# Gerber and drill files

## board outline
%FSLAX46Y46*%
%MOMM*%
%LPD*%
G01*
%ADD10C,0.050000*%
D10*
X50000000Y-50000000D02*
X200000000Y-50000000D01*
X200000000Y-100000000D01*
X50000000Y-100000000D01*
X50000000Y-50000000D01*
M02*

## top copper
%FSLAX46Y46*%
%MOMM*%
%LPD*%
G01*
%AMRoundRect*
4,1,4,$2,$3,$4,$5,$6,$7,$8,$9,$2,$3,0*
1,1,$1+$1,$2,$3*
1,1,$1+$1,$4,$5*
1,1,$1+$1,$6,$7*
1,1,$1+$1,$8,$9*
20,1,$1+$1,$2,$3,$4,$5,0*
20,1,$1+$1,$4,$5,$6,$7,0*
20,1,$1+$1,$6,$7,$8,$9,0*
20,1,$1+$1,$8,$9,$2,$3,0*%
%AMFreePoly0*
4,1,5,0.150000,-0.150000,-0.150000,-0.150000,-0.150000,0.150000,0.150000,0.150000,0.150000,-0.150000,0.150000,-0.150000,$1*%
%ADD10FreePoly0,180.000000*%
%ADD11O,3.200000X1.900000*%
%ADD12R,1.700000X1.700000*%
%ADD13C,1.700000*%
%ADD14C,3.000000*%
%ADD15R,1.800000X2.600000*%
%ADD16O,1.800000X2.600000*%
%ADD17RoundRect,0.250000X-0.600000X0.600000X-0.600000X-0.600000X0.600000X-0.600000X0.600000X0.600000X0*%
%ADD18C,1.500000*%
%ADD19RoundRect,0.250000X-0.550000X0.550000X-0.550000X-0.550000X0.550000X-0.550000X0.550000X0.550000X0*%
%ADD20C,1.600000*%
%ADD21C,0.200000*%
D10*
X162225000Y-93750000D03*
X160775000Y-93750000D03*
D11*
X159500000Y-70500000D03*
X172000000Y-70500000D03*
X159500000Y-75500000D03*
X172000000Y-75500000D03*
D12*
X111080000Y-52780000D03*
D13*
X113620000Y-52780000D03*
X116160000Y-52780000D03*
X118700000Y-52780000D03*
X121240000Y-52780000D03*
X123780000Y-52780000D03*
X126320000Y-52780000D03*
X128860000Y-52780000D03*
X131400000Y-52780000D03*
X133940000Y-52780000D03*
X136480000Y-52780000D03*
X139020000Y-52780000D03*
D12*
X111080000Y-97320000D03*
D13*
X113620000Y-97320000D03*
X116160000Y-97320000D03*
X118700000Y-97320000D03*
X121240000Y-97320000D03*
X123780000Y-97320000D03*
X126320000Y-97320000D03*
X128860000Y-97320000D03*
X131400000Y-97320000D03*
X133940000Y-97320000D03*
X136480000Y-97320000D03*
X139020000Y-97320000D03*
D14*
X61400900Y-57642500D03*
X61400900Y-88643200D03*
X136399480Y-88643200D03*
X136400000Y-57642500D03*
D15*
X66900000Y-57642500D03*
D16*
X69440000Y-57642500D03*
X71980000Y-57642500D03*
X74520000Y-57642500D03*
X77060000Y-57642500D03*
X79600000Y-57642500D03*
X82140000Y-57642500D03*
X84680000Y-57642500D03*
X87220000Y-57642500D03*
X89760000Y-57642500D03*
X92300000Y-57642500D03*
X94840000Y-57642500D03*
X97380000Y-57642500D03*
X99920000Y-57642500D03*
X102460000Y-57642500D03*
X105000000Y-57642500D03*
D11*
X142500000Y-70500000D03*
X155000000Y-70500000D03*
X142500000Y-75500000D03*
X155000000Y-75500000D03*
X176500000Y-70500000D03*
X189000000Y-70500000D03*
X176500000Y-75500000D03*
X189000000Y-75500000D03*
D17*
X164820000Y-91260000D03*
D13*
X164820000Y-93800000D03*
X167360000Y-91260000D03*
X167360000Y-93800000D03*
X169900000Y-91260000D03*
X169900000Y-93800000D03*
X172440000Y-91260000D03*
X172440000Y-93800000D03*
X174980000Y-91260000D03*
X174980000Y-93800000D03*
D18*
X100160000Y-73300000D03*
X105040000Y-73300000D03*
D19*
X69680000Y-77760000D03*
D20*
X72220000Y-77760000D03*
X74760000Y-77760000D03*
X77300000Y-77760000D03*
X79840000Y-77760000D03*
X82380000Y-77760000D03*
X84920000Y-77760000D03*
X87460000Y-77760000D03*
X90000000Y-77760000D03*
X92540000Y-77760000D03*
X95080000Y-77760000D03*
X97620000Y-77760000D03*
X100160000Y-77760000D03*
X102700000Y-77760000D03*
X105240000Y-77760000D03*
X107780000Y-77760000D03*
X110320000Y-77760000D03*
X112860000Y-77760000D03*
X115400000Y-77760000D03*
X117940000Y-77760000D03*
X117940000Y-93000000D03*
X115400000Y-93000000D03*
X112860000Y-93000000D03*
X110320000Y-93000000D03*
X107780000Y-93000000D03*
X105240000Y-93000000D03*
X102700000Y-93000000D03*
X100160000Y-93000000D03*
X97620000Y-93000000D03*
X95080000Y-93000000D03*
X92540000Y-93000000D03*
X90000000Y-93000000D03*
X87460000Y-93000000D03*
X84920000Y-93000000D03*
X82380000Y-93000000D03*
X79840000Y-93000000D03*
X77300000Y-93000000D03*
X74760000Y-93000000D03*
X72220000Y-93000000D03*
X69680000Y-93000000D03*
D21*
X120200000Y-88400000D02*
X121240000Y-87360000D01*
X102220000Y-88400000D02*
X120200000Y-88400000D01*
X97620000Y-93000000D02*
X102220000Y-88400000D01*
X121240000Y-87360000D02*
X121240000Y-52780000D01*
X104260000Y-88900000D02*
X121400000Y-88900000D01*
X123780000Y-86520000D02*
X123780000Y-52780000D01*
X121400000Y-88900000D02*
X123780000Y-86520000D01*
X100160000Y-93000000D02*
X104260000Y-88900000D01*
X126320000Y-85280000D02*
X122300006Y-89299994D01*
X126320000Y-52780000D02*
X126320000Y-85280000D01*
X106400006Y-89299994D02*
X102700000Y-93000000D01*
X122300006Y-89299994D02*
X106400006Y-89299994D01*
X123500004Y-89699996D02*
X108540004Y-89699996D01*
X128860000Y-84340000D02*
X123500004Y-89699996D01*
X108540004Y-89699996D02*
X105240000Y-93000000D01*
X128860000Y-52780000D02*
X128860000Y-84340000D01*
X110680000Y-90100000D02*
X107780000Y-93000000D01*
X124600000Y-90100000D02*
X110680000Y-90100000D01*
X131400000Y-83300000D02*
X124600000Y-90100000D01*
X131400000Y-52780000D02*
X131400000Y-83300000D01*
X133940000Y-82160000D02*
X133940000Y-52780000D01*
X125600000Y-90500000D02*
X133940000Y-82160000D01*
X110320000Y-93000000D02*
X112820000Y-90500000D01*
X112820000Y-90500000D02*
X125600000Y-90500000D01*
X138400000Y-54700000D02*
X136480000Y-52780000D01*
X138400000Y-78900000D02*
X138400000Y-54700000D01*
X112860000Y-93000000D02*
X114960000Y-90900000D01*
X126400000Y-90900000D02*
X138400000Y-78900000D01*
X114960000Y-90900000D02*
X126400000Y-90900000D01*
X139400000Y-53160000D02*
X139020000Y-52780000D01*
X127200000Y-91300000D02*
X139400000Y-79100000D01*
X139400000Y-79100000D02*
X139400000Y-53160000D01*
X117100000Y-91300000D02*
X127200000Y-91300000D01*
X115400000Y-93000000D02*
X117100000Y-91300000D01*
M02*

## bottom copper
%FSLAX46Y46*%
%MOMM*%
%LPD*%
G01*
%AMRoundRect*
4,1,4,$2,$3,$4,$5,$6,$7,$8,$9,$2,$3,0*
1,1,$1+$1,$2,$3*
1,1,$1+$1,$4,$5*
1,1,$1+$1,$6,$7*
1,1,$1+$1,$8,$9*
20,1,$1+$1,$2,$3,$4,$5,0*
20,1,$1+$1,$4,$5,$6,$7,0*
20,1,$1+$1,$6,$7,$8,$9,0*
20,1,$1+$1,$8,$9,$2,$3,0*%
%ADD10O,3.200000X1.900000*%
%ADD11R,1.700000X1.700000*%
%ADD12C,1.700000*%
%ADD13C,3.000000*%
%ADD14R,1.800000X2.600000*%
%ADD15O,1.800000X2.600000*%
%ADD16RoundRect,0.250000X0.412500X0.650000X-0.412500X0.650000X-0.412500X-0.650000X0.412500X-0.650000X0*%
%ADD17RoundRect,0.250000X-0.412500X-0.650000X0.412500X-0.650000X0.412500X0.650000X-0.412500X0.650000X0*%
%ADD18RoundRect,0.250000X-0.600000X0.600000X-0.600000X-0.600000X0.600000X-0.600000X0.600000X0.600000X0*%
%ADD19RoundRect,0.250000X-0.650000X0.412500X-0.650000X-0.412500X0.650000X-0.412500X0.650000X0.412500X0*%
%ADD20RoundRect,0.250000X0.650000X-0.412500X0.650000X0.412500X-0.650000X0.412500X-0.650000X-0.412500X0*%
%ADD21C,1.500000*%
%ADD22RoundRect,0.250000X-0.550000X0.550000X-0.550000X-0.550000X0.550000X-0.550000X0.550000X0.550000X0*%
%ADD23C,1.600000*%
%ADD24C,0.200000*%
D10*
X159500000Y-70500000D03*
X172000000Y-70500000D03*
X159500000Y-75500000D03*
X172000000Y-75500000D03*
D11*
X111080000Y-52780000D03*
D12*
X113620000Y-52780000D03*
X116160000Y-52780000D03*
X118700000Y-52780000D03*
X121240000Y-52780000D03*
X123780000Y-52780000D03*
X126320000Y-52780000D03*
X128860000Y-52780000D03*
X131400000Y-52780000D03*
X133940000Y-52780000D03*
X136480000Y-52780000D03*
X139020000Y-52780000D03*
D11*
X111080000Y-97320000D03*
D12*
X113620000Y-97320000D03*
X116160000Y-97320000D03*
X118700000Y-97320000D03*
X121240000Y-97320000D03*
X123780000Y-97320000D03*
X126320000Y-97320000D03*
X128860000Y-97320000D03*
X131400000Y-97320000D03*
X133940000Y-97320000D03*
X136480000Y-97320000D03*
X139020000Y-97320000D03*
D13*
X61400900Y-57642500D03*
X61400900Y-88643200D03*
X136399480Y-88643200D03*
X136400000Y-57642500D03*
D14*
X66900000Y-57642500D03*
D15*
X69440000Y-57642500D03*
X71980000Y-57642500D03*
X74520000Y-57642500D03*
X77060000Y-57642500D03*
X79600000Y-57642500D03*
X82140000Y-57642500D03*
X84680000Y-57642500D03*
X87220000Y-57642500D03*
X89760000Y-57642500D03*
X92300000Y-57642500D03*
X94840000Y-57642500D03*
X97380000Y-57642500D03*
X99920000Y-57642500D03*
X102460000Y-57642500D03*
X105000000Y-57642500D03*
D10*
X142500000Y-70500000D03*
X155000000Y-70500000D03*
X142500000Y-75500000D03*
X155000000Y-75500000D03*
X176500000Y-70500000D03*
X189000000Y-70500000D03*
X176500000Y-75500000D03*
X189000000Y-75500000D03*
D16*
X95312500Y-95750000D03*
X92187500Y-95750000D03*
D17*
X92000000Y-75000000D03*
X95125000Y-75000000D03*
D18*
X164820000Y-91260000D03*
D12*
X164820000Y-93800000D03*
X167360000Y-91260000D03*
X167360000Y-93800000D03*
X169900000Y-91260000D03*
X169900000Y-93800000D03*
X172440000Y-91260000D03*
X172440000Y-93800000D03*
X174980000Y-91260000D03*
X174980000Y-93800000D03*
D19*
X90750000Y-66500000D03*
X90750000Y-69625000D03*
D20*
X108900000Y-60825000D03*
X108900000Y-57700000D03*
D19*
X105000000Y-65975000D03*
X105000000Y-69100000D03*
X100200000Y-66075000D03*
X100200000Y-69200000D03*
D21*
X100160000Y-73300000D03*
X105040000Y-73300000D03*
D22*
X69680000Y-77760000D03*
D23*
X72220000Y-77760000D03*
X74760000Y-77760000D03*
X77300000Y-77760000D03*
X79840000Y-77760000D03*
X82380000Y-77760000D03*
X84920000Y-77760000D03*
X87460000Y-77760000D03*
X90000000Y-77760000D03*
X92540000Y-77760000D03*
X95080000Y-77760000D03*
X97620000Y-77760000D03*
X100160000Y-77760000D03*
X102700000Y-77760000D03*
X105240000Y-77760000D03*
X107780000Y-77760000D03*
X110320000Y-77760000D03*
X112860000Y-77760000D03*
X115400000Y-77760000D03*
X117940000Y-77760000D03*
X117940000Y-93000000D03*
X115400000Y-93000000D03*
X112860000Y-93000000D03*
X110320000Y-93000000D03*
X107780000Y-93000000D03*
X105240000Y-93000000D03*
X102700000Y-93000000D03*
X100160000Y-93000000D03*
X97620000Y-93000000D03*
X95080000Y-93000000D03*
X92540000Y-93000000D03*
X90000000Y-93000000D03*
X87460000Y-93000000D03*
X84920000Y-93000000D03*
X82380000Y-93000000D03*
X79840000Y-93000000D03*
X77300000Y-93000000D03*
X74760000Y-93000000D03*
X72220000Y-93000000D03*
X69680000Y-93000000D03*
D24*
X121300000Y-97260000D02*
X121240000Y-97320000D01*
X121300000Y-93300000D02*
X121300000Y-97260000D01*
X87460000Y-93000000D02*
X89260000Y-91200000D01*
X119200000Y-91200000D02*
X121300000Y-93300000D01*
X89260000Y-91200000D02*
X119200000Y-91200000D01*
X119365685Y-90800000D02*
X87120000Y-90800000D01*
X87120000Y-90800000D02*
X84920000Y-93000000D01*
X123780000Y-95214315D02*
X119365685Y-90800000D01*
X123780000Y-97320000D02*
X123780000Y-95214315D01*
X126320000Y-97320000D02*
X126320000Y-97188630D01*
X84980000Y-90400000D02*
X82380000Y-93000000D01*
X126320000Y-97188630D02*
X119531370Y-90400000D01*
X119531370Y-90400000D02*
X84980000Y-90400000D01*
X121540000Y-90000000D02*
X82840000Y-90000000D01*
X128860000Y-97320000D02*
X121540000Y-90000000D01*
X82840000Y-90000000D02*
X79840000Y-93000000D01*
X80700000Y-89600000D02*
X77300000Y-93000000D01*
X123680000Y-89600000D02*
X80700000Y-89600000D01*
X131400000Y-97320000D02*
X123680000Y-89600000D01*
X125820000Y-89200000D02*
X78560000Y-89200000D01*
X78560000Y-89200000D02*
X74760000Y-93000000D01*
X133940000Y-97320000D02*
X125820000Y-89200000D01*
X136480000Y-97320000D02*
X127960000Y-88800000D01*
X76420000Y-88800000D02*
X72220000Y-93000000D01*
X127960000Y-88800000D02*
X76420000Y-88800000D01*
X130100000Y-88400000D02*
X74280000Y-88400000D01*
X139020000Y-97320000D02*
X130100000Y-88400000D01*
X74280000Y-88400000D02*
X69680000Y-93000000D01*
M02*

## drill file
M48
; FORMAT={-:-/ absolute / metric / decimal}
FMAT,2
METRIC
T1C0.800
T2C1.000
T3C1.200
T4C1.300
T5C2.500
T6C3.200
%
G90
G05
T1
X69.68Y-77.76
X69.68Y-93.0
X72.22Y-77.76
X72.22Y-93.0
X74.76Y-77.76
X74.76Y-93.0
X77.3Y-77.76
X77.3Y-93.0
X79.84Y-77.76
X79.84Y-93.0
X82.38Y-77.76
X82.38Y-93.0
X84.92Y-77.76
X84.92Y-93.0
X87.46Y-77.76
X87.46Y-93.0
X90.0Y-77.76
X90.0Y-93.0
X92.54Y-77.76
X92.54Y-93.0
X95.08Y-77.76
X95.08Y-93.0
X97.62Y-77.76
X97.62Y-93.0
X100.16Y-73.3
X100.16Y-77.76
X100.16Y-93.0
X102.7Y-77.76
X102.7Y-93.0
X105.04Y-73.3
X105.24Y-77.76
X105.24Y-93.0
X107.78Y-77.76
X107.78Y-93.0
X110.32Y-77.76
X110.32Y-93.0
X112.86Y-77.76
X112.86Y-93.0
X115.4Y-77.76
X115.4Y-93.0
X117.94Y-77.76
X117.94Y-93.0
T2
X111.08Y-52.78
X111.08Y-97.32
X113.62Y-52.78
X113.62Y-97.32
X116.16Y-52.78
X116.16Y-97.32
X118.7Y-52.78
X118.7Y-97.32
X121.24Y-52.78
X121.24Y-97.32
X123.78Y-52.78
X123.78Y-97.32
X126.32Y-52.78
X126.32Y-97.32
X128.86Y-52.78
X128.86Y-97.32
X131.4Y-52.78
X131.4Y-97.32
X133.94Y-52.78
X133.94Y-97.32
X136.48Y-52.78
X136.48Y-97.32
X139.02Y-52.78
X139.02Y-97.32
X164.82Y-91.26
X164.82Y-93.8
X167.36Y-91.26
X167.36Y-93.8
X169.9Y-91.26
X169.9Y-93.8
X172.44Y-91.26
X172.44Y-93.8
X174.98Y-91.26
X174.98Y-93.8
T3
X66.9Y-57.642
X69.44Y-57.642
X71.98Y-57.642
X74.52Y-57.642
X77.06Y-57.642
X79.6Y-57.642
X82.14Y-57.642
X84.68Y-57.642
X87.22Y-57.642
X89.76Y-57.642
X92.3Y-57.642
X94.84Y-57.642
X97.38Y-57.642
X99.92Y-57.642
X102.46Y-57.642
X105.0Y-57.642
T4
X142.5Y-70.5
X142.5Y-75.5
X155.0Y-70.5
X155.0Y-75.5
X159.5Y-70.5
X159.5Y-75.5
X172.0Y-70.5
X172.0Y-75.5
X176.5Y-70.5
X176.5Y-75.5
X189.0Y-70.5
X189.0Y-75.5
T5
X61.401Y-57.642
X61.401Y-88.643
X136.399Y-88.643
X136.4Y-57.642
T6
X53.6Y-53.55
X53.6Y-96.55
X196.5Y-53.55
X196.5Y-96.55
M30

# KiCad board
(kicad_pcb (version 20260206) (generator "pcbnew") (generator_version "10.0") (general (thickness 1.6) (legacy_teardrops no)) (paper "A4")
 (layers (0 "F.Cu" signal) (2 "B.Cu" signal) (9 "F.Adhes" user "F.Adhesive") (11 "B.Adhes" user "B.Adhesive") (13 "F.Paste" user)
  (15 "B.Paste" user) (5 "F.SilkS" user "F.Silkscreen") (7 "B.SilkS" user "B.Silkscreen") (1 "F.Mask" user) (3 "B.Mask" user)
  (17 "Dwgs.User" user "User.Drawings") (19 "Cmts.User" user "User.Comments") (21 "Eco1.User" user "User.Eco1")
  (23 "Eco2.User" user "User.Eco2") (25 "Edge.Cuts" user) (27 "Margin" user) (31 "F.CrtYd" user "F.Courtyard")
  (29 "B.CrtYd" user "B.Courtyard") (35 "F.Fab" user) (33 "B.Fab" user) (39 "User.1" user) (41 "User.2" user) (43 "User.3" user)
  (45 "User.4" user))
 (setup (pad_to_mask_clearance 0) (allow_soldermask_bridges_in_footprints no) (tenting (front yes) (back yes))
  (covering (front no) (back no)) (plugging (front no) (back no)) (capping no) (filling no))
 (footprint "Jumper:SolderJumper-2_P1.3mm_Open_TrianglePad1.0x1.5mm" (layer "F.Cu") (at 161.5 93.75 180)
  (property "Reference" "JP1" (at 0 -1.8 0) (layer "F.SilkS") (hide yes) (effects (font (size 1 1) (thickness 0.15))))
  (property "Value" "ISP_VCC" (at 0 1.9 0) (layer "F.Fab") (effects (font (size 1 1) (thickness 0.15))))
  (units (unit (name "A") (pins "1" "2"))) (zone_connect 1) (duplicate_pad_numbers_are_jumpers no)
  (pad "1" smd custom (at -0.725 0 180) (size 0.3 0.3) (layers "F.Cu" "F.Mask") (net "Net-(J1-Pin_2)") (zone_connect 2)
   (thermal_bridge_angle 45) (options (clearance outline) (anchor rect)) (primitives))
  (pad "2" smd custom (at 0.725 0 180) (size 0.3 0.3) (layers "F.Cu" "F.Mask") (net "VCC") (zone_connect 2) (thermal_bridge_angle 45)
   (options (clearance outline) (anchor rect)) (primitives)))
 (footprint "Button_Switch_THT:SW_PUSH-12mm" (layer "F.Cu") (at 159.5 70.5)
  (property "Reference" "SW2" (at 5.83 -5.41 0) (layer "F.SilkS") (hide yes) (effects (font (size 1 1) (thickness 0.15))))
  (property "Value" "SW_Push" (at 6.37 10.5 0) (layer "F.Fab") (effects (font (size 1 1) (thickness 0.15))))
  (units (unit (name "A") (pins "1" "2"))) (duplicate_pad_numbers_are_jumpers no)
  (pad "1" thru_hole oval (at 0 0) (size 3.2 1.9) (drill 1.3) (layers "*.Cu" "*.Mask") (remove_unused_layers no) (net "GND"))
  (pad "1" thru_hole oval (at 12.5 0) (size 3.2 1.9) (drill 1.3) (layers "*.Cu" "*.Mask") (remove_unused_layers no) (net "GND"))
  (pad "2" thru_hole oval (at 0 5) (size 3.2 1.9) (drill 1.3) (layers "*.Cu" "*.Mask") (remove_unused_layers no) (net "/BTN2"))
  (pad "2" thru_hole oval (at 12.5 5) (size 3.2 1.9) (drill 1.3) (layers "*.Cu" "*.Mask") (remove_unused_layers no) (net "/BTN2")))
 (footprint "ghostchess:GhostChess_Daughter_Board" (layer "F.Cu") (at 125.05 75.05)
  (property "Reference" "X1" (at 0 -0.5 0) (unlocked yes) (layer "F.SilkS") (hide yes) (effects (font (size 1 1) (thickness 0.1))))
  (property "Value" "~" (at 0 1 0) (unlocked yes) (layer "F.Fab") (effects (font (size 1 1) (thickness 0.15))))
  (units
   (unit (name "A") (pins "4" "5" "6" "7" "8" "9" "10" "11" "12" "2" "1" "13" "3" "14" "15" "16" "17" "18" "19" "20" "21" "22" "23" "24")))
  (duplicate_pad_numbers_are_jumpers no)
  (pad "" np_thru_hole circle (at -71.45 -21.5) (size 3.2 3.2) (drill 3.2) (layers "*.Cu" "*.Mask"))
  (pad "" np_thru_hole circle (at -71.45 21.5) (size 3.2 3.2) (drill 3.2) (layers "*.Cu" "*.Mask"))
  (pad "" np_thru_hole circle (at 71.45 -21.5) (size 3.2 3.2) (drill 3.2) (layers "*.Cu" "*.Mask"))
  (pad "" np_thru_hole circle (at 71.45 21.5) (size 3.2 3.2) (drill 3.2) (layers "*.Cu" "*.Mask"))
  (pad "1" thru_hole rect (at -13.97 -22.27 90) (size 1.7 1.7) (drill 1) (layers "*.Cu" "*.Mask") (remove_unused_layers no) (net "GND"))
  (pad "2" thru_hole circle (at -11.43 -22.27 90) (size 1.7 1.7) (drill 1) (layers "*.Cu" "*.Mask") (remove_unused_layers no) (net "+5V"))
  (pad "3" thru_hole circle (at -8.89 -22.27 90) (size 1.7 1.7) (drill 1) (layers "*.Cu" "*.Mask") (remove_unused_layers no) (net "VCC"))
  (pad "4" thru_hole circle (at -6.35 -22.27 90) (size 1.7 1.7) (drill 1) (layers "*.Cu" "*.Mask") (remove_unused_layers no) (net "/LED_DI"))
  (pad "5" thru_hole circle (at -3.81 -22.27 90) (size 1.7 1.7) (drill 1) (layers "*.Cu" "*.Mask") (remove_unused_layers no)
   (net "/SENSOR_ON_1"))
  (pad "6" thru_hole circle (at -1.27 -22.27 90) (size 1.7 1.7) (drill 1) (layers "*.Cu" "*.Mask") (remove_unused_layers no)
   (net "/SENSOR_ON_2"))
  (pad "7" thru_hole circle (at 1.27 -22.27 90) (size 1.7 1.7) (drill 1) (layers "*.Cu" "*.Mask") (remove_unused_layers no)
   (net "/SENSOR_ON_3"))
  (pad "8" thru_hole circle (at 3.81 -22.27 90) (size 1.7 1.7) (drill 1) (layers "*.Cu" "*.Mask") (remove_unused_layers no)
   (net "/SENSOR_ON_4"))
  (pad "9" thru_hole circle (at 6.35 -22.27 90) (size 1.7 1.7) (drill 1) (layers "*.Cu" "*.Mask") (remove_unused_layers no)
   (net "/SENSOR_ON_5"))
  (pad "10" thru_hole circle (at 8.89 -22.27 90) (size 1.7 1.7) (drill 1) (layers "*.Cu" "*.Mask") (remove_unused_layers no)
   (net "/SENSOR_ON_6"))
  (pad "11" thru_hole circle (at 11.43 -22.27 90) (size 1.7 1.7) (drill 1) (layers "*.Cu" "*.Mask") (remove_unused_layers no)
   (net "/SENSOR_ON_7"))
  (pad "12" thru_hole circle (at 13.97 -22.27 90) (size 1.7 1.7) (drill 1) (layers "*.Cu" "*.Mask") (remove_unused_layers no)
   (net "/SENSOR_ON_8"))
  (pad "13" thru_hole rect (at -13.97 22.27 90) (size 1.7 1.7) (drill 1) (layers "*.Cu" "*.Mask") (remove_unused_layers no) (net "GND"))
  (pad "14" thru_hole circle (at -11.43 22.27 90) (size 1.7 1.7) (drill 1) (layers "*.Cu" "*.Mask") (remove_unused_layers no) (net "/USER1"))
  (pad "15" thru_hole circle (at -8.89 22.27 90) (size 1.7 1.7) (drill 1) (layers "*.Cu" "*.Mask") (remove_unused_layers no) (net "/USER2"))
  (pad "16" thru_hole circle (at -6.35 22.27 90) (size 1.7 1.7) (drill 1) (layers "*.Cu" "*.Mask") (remove_unused_layers no) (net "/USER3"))
  (pad "17" thru_hole circle (at -3.81 22.27 90) (size 1.7 1.7) (drill 1) (layers "*.Cu" "*.Mask") (remove_unused_layers no)
   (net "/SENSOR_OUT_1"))
  (pad "18" thru_hole circle (at -1.27 22.27 90) (size 1.7 1.7) (drill 1) (layers "*.Cu" "*.Mask") (remove_unused_layers no)
   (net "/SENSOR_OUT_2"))
  (pad "19" thru_hole circle (at 1.27 22.27 90) (size 1.7 1.7) (drill 1) (layers "*.Cu" "*.Mask") (remove_unused_layers no)
   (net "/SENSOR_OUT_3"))
  (pad "20" thru_hole circle (at 3.81 22.27 90) (size 1.7 1.7) (drill 1) (layers "*.Cu" "*.Mask") (remove_unused_layers no)
   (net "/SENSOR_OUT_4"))
  (pad "21" thru_hole circle (at 6.35 22.27 90) (size 1.7 1.7) (drill 1) (layers "*.Cu" "*.Mask") (remove_unused_layers no)
   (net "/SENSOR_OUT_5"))
  (pad "22" thru_hole circle (at 8.89 22.27 90) (size 1.7 1.7) (drill 1) (layers "*.Cu" "*.Mask") (remove_unused_layers no)
   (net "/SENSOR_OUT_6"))
  (pad "23" thru_hole circle (at 11.43 22.27 90) (size 1.7 1.7) (drill 1) (layers "*.Cu" "*.Mask") (remove_unused_layers no)
   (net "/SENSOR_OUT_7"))
  (pad "24" thru_hole circle (at 13.97 22.27 90) (size 1.7 1.7) (drill 1) (layers "*.Cu" "*.Mask") (remove_unused_layers no)
   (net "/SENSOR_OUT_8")))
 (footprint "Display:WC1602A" (layer "F.Cu") (at 66.9 57.6425)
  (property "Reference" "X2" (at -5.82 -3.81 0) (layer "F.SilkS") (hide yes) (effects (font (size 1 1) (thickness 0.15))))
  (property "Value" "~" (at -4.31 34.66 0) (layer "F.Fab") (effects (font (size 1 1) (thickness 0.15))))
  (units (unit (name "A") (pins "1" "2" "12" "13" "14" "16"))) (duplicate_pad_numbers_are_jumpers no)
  (pad "" thru_hole circle (at -5.4991 0) (size 3 3) (drill 2.5) (layers "*.Cu" "*.Mask") (remove_unused_layers no))
  (pad "" thru_hole circle (at -5.4991 31.0007) (size 3 3) (drill 2.5) (layers "*.Cu" "*.Mask") (remove_unused_layers no))
  (pad "" thru_hole circle (at 69.49948 31.0007) (size 3 3) (drill 2.5) (layers "*.Cu" "*.Mask") (remove_unused_layers no))
  (pad "" thru_hole circle (at 69.5 0) (size 3 3) (drill 2.5) (layers "*.Cu" "*.Mask") (remove_unused_layers no))
  (pad "1" thru_hole rect (at 0 0) (size 1.8 2.6) (drill 1.2) (layers "*.Cu" "*.Mask") (remove_unused_layers no) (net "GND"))
  (pad "2" thru_hole oval (at 2.54 0) (size 1.8 2.6) (drill 1.2) (layers "*.Cu" "*.Mask") (remove_unused_layers no) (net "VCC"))
  (pad "3" thru_hole oval (at 5.08 0) (size 1.8 2.6) (drill 1.2) (layers "*.Cu" "*.Mask") (remove_unused_layers no))
  (pad "4" thru_hole oval (at 7.62 0) (size 1.8 2.6) (drill 1.2) (layers "*.Cu" "*.Mask") (remove_unused_layers no))
  (pad "5" thru_hole oval (at 10.16 0) (size 1.8 2.6) (drill 1.2) (layers "*.Cu" "*.Mask") (remove_unused_layers no))
  (pad "6" thru_hole oval (at 12.7 0) (size 1.8 2.6) (drill 1.2) (layers "*.Cu" "*.Mask") (remove_unused_layers no))
  (pad "7" thru_hole oval (at 15.24 0) (size 1.8 2.6) (drill 1.2) (layers "*.Cu" "*.Mask") (remove_unused_layers no))
  (pad "8" thru_hole oval (at 17.78 0) (size 1.8 2.6) (drill 1.2) (layers "*.Cu" "*.Mask") (remove_unused_layers no))
  (pad "9" thru_hole oval (at 20.32 0) (size 1.8 2.6) (drill 1.2) (layers "*.Cu" "*.Mask") (remove_unused_layers no))
  (pad "10" thru_hole oval (at 22.86 0) (size 1.8 2.6) (drill 1.2) (layers "*.Cu" "*.Mask") (remove_unused_layers no))
  (pad "11" thru_hole oval (at 25.4 0) (size 1.8 2.6) (drill 1.2) (layers "*.Cu" "*.Mask") (remove_unused_layers no))
  (pad "12" thru_hole oval (at 27.94 0) (size 1.8 2.6) (drill 1.2) (layers "*.Cu" "*.Mask") (remove_unused_layers no) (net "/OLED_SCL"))
  (pad "13" thru_hole oval (at 30.48 0) (size 1.8 2.6) (drill 1.2) (layers "*.Cu" "*.Mask") (remove_unused_layers no)
   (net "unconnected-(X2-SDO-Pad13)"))
  (pad "14" thru_hole oval (at 33.02 0) (size 1.8 2.6) (drill 1.2) (layers "*.Cu" "*.Mask") (remove_unused_layers no) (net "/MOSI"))
  (pad "15" thru_hole oval (at 35.56 0) (size 1.8 2.6) (drill 1.2) (layers "*.Cu" "*.Mask") (remove_unused_layers no))
  (pad "16" thru_hole oval (at 38.1 0) (size 1.8 2.6) (drill 1.2) (layers "*.Cu" "*.Mask") (remove_unused_layers no) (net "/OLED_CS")))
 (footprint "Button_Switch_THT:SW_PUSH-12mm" (layer "F.Cu") (at 142.5 70.5)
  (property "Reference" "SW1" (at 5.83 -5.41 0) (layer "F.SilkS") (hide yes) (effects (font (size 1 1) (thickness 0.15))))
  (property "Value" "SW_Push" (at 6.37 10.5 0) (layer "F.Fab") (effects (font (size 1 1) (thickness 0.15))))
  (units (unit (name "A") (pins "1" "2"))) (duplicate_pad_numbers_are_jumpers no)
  (pad "1" thru_hole oval (at 0 0) (size 3.2 1.9) (drill 1.3) (layers "*.Cu" "*.Mask") (remove_unused_layers no) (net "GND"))
  (pad "1" thru_hole oval (at 12.5 0) (size 3.2 1.9) (drill 1.3) (layers "*.Cu" "*.Mask") (remove_unused_layers no) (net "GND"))
  (pad "2" thru_hole oval (at 0 5) (size 3.2 1.9) (drill 1.3) (layers "*.Cu" "*.Mask") (remove_unused_layers no) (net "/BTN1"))
  (pad "2" thru_hole oval (at 12.5 5) (size 3.2 1.9) (drill 1.3) (layers "*.Cu" "*.Mask") (remove_unused_layers no) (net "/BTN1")))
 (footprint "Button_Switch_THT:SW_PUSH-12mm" (layer "F.Cu") (at 176.5 70.5)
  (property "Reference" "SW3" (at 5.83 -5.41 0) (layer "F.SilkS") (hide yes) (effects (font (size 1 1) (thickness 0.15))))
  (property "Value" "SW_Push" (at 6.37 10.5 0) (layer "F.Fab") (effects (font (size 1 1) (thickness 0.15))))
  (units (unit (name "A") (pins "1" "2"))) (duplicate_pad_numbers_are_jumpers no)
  (pad "1" thru_hole oval (at 0 0) (size 3.2 1.9) (drill 1.3) (layers "*.Cu" "*.Mask") (remove_unused_layers no) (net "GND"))
  (pad "1" thru_hole oval (at 12.5 0) (size 3.2 1.9) (drill 1.3) (layers "*.Cu" "*.Mask") (remove_unused_layers no) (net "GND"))
  (pad "2" thru_hole oval (at 0 5) (size 3.2 1.9) (drill 1.3) (layers "*.Cu" "*.Mask") (remove_unused_layers no) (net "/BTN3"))
  (pad "2" thru_hole oval (at 12.5 5) (size 3.2 1.9) (drill 1.3) (layers "*.Cu" "*.Mask") (remove_unused_layers no) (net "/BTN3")))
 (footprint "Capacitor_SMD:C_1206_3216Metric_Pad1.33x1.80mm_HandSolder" (layer "B.Cu") (at 93.75 95.75 180)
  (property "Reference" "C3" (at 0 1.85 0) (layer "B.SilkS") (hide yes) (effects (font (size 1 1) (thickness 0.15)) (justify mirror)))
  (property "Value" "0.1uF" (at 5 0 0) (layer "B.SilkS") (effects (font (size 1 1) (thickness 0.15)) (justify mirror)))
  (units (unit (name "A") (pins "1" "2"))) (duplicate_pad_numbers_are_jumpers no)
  (pad "1" smd roundrect (at -1.5625 0 180) (size 1.325 1.8) (layers "B.Cu" "B.Mask" "B.Paste") (roundrect_rratio 0.188679) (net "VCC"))
  (pad "2" smd roundrect (at 1.5625 0 180) (size 1.325 1.8) (layers "B.Cu" "B.Mask" "B.Paste") (roundrect_rratio 0.188679) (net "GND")))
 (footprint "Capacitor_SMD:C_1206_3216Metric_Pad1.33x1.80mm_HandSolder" (layer "B.Cu") (at 93.5625 75)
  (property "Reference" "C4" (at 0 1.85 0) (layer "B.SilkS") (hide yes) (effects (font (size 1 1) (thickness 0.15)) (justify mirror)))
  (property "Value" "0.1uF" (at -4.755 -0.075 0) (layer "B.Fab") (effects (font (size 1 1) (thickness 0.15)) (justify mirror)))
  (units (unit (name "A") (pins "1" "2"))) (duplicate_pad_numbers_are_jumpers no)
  (pad "1" smd roundrect (at -1.5625 0) (size 1.325 1.8) (layers "B.Cu" "B.Mask" "B.Paste") (roundrect_rratio 0.188679) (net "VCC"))
  (pad "2" smd roundrect (at 1.5625 0) (size 1.325 1.8) (layers "B.Cu" "B.Mask" "B.Paste") (roundrect_rratio 0.188679) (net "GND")))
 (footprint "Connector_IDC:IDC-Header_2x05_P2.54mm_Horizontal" (layer "B.Cu") (at 164.82 91.26 -90)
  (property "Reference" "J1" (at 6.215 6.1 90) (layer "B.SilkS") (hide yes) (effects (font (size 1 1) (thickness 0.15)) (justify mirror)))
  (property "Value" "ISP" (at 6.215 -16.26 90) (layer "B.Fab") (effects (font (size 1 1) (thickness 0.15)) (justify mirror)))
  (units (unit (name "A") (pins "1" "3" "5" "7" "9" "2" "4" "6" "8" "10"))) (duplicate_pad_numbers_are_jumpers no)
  (pad "1" thru_hole roundrect (at 0 0 270) (size 1.7 1.7) (drill 1) (layers "*.Cu" "*.Mask") (remove_unused_layers no)
   (roundrect_rratio 0.147059) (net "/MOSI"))
  (pad "2" thru_hole circle (at 2.54 0 270) (size 1.7 1.7) (drill 1) (layers "*.Cu" "*.Mask") (remove_unused_layers no)
   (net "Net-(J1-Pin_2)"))
  (pad "3" thru_hole circle (at 0 -2.54 270) (size 1.7 1.7) (drill 1) (layers "*.Cu" "*.Mask") (remove_unused_layers no)
   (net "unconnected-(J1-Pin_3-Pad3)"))
  (pad "4" thru_hole circle (at 2.54 -2.54 270) (size 1.7 1.7) (drill 1) (layers "*.Cu" "*.Mask") (remove_unused_layers no) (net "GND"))
  (pad "5" thru_hole circle (at 0 -5.08 270) (size 1.7 1.7) (drill 1) (layers "*.Cu" "*.Mask") (remove_unused_layers no) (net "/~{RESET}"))
  (pad "6" thru_hole circle (at 2.54 -5.08 270) (size 1.7 1.7) (drill 1) (layers "*.Cu" "*.Mask") (remove_unused_layers no) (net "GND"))
  (pad "7" thru_hole circle (at 0 -7.62 270) (size 1.7 1.7) (drill 1) (layers "*.Cu" "*.Mask") (remove_unused_layers no) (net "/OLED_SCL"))
  (pad "8" thru_hole circle (at 2.54 -7.62 270) (size 1.7 1.7) (drill 1) (layers "*.Cu" "*.Mask") (remove_unused_layers no) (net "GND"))
  (pad "9" thru_hole circle (at 0 -10.16 270) (size 1.7 1.7) (drill 1) (layers "*.Cu" "*.Mask") (remove_unused_layers no) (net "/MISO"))
  (pad "10" thru_hole circle (at 2.54 -10.16 270) (size 1.7 1.7) (drill 1) (layers "*.Cu" "*.Mask") (remove_unused_layers no) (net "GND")))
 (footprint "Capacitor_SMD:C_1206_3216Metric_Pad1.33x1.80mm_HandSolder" (layer "B.Cu") (at 90.75 68.0625 -90)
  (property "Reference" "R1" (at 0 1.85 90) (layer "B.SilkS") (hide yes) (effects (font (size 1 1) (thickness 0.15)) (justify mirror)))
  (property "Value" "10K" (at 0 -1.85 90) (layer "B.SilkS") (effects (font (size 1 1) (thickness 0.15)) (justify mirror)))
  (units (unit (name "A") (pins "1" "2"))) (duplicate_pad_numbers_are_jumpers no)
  (pad "1" smd roundrect (at -1.5625 0 270) (size 1.325 1.8) (layers "B.Cu" "B.Mask" "B.Paste") (roundrect_rratio 0.188679) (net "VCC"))
  (pad "2" smd roundrect (at 1.5625 0 270) (size 1.325 1.8) (layers "B.Cu" "B.Mask" "B.Paste") (roundrect_rratio 0.188679) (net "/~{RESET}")))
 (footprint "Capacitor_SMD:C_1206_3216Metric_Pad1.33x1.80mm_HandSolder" (layer "B.Cu") (at 108.9 59.2625 90)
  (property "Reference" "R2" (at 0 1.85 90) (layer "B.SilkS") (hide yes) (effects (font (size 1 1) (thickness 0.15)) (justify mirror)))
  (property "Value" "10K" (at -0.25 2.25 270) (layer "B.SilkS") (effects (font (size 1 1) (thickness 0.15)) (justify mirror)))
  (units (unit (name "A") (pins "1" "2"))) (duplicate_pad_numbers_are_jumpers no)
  (pad "1" smd roundrect (at -1.5625 0 90) (size 1.325 1.8) (layers "B.Cu" "B.Mask" "B.Paste") (roundrect_rratio 0.188679) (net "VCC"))
  (pad "2" smd roundrect (at 1.5625 0 90) (size 1.325 1.8) (layers "B.Cu" "B.Mask" "B.Paste") (roundrect_rratio 0.188679) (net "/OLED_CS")))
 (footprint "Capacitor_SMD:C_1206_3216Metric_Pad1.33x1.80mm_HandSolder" (layer "B.Cu") (at 105 67.5375 -90)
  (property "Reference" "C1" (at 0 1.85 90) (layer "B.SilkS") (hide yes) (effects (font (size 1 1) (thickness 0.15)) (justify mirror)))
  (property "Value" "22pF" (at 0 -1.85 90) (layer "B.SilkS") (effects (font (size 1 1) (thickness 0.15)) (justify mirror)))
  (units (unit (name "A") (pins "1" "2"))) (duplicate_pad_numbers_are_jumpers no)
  (pad "1" smd roundrect (at -1.5625 0 270) (size 1.325 1.8) (layers "B.Cu" "B.Mask" "B.Paste") (roundrect_rratio 0.188679) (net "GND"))
  (pad "2" smd roundrect (at 1.5625 0 270) (size 1.325 1.8) (layers "B.Cu" "B.Mask" "B.Paste") (roundrect_rratio 0.188679)
   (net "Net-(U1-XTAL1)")))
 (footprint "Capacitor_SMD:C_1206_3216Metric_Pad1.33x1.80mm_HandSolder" (layer "B.Cu") (at 100.2 67.6375 -90)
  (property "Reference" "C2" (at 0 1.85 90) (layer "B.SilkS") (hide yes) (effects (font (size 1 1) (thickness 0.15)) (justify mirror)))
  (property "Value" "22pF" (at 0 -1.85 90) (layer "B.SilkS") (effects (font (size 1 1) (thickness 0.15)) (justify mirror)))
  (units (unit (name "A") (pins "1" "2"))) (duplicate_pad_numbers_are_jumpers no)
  (pad "1" smd roundrect (at -1.5625 0 270) (size 1.325 1.8) (layers "B.Cu" "B.Mask" "B.Paste") (roundrect_rratio 0.188679) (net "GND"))
  (pad "2" smd roundrect (at 1.5625 0 270) (size 1.325 1.8) (layers "B.Cu" "B.Mask" "B.Paste") (roundrect_rratio 0.188679)
   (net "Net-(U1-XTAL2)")))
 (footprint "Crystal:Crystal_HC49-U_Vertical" (layer "B.Cu") (at 100.16 73.3)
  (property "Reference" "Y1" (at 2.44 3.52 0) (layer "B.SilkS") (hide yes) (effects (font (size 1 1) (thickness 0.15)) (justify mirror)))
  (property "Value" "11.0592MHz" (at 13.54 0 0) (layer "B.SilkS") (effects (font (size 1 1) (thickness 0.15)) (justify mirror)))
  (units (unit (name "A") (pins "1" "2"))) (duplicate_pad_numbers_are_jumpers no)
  (pad "1" thru_hole circle (at 0 0) (size 1.5 1.5) (drill 0.8) (layers "*.Cu" "*.Mask") (remove_unused_layers no) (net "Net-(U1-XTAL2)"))
  (pad "2" thru_hole circle (at 4.88 0) (size 1.5 1.5) (drill 0.8) (layers "*.Cu" "*.Mask") (remove_unused_layers no) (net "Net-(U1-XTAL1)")))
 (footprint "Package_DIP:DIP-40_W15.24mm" (layer "B.Cu") (at 69.68 77.76 -90)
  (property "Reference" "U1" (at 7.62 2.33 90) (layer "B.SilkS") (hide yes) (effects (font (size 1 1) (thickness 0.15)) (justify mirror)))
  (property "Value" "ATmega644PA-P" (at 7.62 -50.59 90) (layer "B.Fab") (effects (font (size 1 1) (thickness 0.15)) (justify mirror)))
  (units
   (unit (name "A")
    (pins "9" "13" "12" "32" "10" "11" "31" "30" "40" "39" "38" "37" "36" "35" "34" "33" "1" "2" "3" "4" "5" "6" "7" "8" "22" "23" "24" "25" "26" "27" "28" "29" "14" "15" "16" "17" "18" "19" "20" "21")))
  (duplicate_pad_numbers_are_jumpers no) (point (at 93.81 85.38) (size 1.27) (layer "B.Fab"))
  (pad "1" thru_hole roundrect (at 0 0 270) (size 1.6 1.6) (drill 0.8) (layers "*.Cu" "*.Mask") (remove_unused_layers no)
   (roundrect_rratio 0.15625) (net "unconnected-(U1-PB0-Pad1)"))
  (pad "2" thru_hole circle (at 0 -2.54 270) (size 1.6 1.6) (drill 0.8) (layers "*.Cu" "*.Mask") (remove_unused_layers no)
   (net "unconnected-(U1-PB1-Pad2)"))
  (pad "3" thru_hole circle (at 0 -5.08 270) (size 1.6 1.6) (drill 0.8) (layers "*.Cu" "*.Mask") (remove_unused_layers no)
   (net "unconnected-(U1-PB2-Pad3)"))
  (pad "4" thru_hole circle (at 0 -7.62 270) (size 1.6 1.6) (drill 0.8) (layers "*.Cu" "*.Mask") (remove_unused_layers no)
   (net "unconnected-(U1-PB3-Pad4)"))
  (pad "5" thru_hole circle (at 0 -10.16 270) (size 1.6 1.6) (drill 0.8) (layers "*.Cu" "*.Mask") (remove_unused_layers no) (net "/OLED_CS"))
  (pad "6" thru_hole circle (at 0 -12.7 270) (size 1.6 1.6) (drill 0.8) (layers "*.Cu" "*.Mask") (remove_unused_layers no) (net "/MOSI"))
  (pad "7" thru_hole circle (at 0 -15.24 270) (size 1.6 1.6) (drill 0.8) (layers "*.Cu" "*.Mask") (remove_unused_layers no) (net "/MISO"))
  (pad "8" thru_hole circle (at 0 -17.78 270) (size 1.6 1.6) (drill 0.8) (layers "*.Cu" "*.Mask") (remove_unused_layers no)
   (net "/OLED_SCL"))
  (pad "9" thru_hole circle (at 0 -20.32 270) (size 1.6 1.6) (drill 0.8) (layers "*.Cu" "*.Mask") (remove_unused_layers no)
   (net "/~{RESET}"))
  (pad "10" thru_hole circle (at 0 -22.86 270) (size 1.6 1.6) (drill 0.8) (layers "*.Cu" "*.Mask") (remove_unused_layers no) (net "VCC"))
  (pad "11" thru_hole circle (at 0 -25.4 270) (size 1.6 1.6) (drill 0.8) (layers "*.Cu" "*.Mask") (remove_unused_layers no) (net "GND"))
  (pad "12" thru_hole circle (at 0 -27.94 270) (size 1.6 1.6) (drill 0.8) (layers "*.Cu" "*.Mask") (remove_unused_layers no)
   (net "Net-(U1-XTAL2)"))
  (pad "13" thru_hole circle (at 0 -30.48 270) (size 1.6 1.6) (drill 0.8) (layers "*.Cu" "*.Mask") (remove_unused_layers no)
   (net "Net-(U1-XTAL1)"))
  (pad "14" thru_hole circle (at 0 -33.02 270) (size 1.6 1.6) (drill 0.8) (layers "*.Cu" "*.Mask") (remove_unused_layers no) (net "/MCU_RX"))
  (pad "15" thru_hole circle (at 0 -35.56 270) (size 1.6 1.6) (drill 0.8) (layers "*.Cu" "*.Mask") (remove_unused_layers no) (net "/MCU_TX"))
  (pad "16" thru_hole circle (at 0 -38.1 270) (size 1.6 1.6) (drill 0.8) (layers "*.Cu" "*.Mask") (remove_unused_layers no) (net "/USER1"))
  (pad "17" thru_hole circle (at 0 -40.64 270) (size 1.6 1.6) (drill 0.8) (layers "*.Cu" "*.Mask") (remove_unused_layers no) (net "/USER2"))
  (pad "18" thru_hole circle (at 0 -43.18 270) (size 1.6 1.6) (drill 0.8) (layers "*.Cu" "*.Mask") (remove_unused_layers no) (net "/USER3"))
  (pad "19" thru_hole circle (at 0 -45.72 270) (size 1.6 1.6) (drill 0.8) (layers "*.Cu" "*.Mask") (remove_unused_layers no) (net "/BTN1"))
  (pad "20" thru_hole circle (at 0 -48.26 270) (size 1.6 1.6) (drill 0.8) (layers "*.Cu" "*.Mask") (remove_unused_layers no) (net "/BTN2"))
  (pad "21" thru_hole circle (at 15.24 -48.26 270) (size 1.6 1.6) (drill 0.8) (layers "*.Cu" "*.Mask") (remove_unused_layers no)
   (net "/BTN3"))
  (pad "22" thru_hole circle (at 15.24 -45.72 270) (size 1.6 1.6) (drill 0.8) (layers "*.Cu" "*.Mask") (remove_unused_layers no)
   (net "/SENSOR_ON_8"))
  (pad "23" thru_hole circle (at 15.24 -43.18 270) (size 1.6 1.6) (drill 0.8) (layers "*.Cu" "*.Mask") (remove_unused_layers no)
   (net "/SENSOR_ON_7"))
  (pad "24" thru_hole circle (at 15.24 -40.64 270) (size 1.6 1.6) (drill 0.8) (layers "*.Cu" "*.Mask") (remove_unused_layers no)
   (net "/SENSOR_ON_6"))
  (pad "25" thru_hole circle (at 15.24 -38.1 270) (size 1.6 1.6) (drill 0.8) (layers "*.Cu" "*.Mask") (remove_unused_layers no)
   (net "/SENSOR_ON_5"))
  (pad "26" thru_hole circle (at 15.24 -35.56 270) (size 1.6 1.6) (drill 0.8) (layers "*.Cu" "*.Mask") (remove_unused_layers no)
   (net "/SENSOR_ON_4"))
  (pad "27" thru_hole circle (at 15.24 -33.02 270) (size 1.6 1.6) (drill 0.8) (layers "*.Cu" "*.Mask") (remove_unused_layers no)
   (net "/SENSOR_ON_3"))
  (pad "28" thru_hole circle (at 15.24 -30.48 270) (size 1.6 1.6) (drill 0.8) (layers "*.Cu" "*.Mask") (remove_unused_layers no)
   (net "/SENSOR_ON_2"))
  (pad "29" thru_hole circle (at 15.24 -27.94 270) (size 1.6 1.6) (drill 0.8) (layers "*.Cu" "*.Mask") (remove_unused_layers no)
   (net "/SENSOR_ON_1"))
  (pad "30" thru_hole circle (at 15.24 -25.4 270) (size 1.6 1.6) (drill 0.8) (layers "*.Cu" "*.Mask") (remove_unused_layers no) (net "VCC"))
  (pad "31" thru_hole circle (at 15.24 -22.86 270) (size 1.6 1.6) (drill 0.8) (layers "*.Cu" "*.Mask") (remove_unused_layers no) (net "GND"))
  (pad "32" thru_hole circle (at 15.24 -20.32 270) (size 1.6 1.6) (drill 0.8) (layers "*.Cu" "*.Mask") (remove_unused_layers no)
   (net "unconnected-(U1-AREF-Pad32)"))
  (pad "33" thru_hole circle (at 15.24 -17.78 270) (size 1.6 1.6) (drill 0.8) (layers "*.Cu" "*.Mask") (remove_unused_layers no)
   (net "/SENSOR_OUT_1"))
  (pad "34" thru_hole circle (at 15.24 -15.24 270) (size 1.6 1.6) (drill 0.8) (layers "*.Cu" "*.Mask") (remove_unused_layers no)
   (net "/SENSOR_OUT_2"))
  (pad "35" thru_hole circle (at 15.24 -12.7 270) (size 1.6 1.6) (drill 0.8) (layers "*.Cu" "*.Mask") (remove_unused_layers no)
   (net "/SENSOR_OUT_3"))
  (pad "36" thru_hole circle (at 15.24 -10.16 270) (size 1.6 1.6) (drill 0.8) (layers "*.Cu" "*.Mask") (remove_unused_layers no)
   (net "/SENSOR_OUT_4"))
  (pad "37" thru_hole circle (at 15.24 -7.62 270) (size 1.6 1.6) (drill 0.8) (layers "*.Cu" "*.Mask") (remove_unused_layers no)
   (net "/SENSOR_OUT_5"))
  (pad "38" thru_hole circle (at 15.24 -5.08 270) (size 1.6 1.6) (drill 0.8) (layers "*.Cu" "*.Mask") (remove_unused_layers no)
   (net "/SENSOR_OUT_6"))
  (pad "39" thru_hole circle (at 15.24 -2.54 270) (size 1.6 1.6) (drill 0.8) (layers "*.Cu" "*.Mask") (remove_unused_layers no)
   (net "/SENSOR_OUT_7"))
  (pad "40" thru_hole circle (at 15.24 0 270) (size 1.6 1.6) (drill 0.8) (layers "*.Cu" "*.Mask") (remove_unused_layers no)
   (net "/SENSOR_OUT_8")))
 (gr_rect (start 50 50) (end 200 100) (stroke (width 0.05) (type default)) (fill no) (layer "Edge.Cuts"))
 (segment (start 120.2 88.4) (end 121.24 87.36) (width 0.2) (layer "F.Cu") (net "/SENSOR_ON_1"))
 (segment (start 102.22 88.4) (end 120.2 88.4) (width 0.2) (layer "F.Cu") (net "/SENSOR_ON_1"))
 (segment (start 97.62 93) (end 102.22 88.4) (width 0.2) (layer "F.Cu") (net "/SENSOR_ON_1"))
 (segment (start 121.24 87.36) (end 121.24 52.78) (width 0.2) (layer "F.Cu") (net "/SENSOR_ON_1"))
 (segment (start 104.26 88.9) (end 121.4 88.9) (width 0.2) (layer "F.Cu") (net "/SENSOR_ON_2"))
 (segment (start 123.78 86.52) (end 123.78 52.78) (width 0.2) (layer "F.Cu") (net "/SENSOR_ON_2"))
 (segment (start 121.4 88.9) (end 123.78 86.52) (width 0.2) (layer "F.Cu") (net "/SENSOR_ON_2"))
 (segment (start 100.16 93) (end 104.26 88.9) (width 0.2) (layer "F.Cu") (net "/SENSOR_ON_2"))
 (segment (start 126.32 85.28) (end 122.300006 89.299994) (width 0.2) (layer "F.Cu") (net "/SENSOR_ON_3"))
 (segment (start 126.32 52.78) (end 126.32 85.28) (width 0.2) (layer "F.Cu") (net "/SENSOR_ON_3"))
 (segment (start 106.400006 89.299994) (end 102.7 93) (width 0.2) (layer "F.Cu") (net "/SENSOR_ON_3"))
 (segment (start 122.300006 89.299994) (end 106.400006 89.299994) (width 0.2) (layer "F.Cu") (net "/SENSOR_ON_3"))
 (segment (start 123.500004 89.699996) (end 108.540004 89.699996) (width 0.2) (layer "F.Cu") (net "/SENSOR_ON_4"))
 (segment (start 128.86 84.34) (end 123.500004 89.699996) (width 0.2) (layer "F.Cu") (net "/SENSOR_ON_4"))
 (segment (start 108.540004 89.699996) (end 105.24 93) (width 0.2) (layer "F.Cu") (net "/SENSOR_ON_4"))
 (segment (start 128.86 52.78) (end 128.86 84.34) (width 0.2) (layer "F.Cu") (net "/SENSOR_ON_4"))
 (segment (start 110.68 90.1) (end 107.78 93) (width 0.2) (layer "F.Cu") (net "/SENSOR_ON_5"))
 (segment (start 124.6 90.1) (end 110.68 90.1) (width 0.2) (layer "F.Cu") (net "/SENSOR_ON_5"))
 (segment (start 131.4 83.3) (end 124.6 90.1) (width 0.2) (layer "F.Cu") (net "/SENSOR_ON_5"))
 (segment (start 131.4 52.78) (end 131.4 83.3) (width 0.2) (layer "F.Cu") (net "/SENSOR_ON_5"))
 (segment (start 133.94 82.16) (end 133.94 52.78) (width 0.2) (layer "F.Cu") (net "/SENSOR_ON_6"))
 (segment (start 125.6 90.5) (end 133.94 82.16) (width 0.2) (layer "F.Cu") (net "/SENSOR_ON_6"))
 (segment (start 110.32 93) (end 112.82 90.5) (width 0.2) (layer "F.Cu") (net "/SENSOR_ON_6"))
 (segment (start 112.82 90.5) (end 125.6 90.5) (width 0.2) (layer "F.Cu") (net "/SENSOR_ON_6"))
 (segment (start 138.4 54.7) (end 136.48 52.78) (width 0.2) (layer "F.Cu") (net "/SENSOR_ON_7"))
 (segment (start 138.4 78.9) (end 138.4 54.7) (width 0.2) (layer "F.Cu") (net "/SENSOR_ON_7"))
 (segment (start 112.86 93) (end 114.96 90.9) (width 0.2) (layer "F.Cu") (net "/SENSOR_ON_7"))
 (segment (start 126.4 90.9) (end 138.4 78.9) (width 0.2) (layer "F.Cu") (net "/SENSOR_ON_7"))
 (segment (start 114.96 90.9) (end 126.4 90.9) (width 0.2) (layer "F.Cu") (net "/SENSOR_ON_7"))
 (segment (start 139.4 53.16) (end 139.02 52.78) (width 0.2) (layer "F.Cu") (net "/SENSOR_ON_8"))
 (segment (start 127.2 91.3) (end 139.4 79.1) (width 0.2) (layer "F.Cu") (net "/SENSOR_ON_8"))
 (segment (start 139.4 79.1) (end 139.4 53.16) (width 0.2) (layer "F.Cu") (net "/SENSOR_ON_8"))
 (segment (start 117.1 91.3) (end 127.2 91.3) (width 0.2) (layer "F.Cu") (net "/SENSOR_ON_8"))
 (segment (start 115.4 93) (end 117.1 91.3) (width 0.2) (layer "F.Cu") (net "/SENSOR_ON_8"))
 (segment (start 121.3 97.26) (end 121.24 97.32) (width 0.2) (layer "B.Cu") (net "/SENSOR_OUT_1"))
 (segment (start 121.3 93.3) (end 121.3 97.26) (width 0.2) (layer "B.Cu") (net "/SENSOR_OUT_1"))
 (segment (start 87.46 93) (end 89.26 91.2) (width 0.2) (layer "B.Cu") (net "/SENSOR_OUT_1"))
 (segment (start 119.2 91.2) (end 121.3 93.3) (width 0.2) (layer "B.Cu") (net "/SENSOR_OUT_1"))
 (segment (start 89.26 91.2) (end 119.2 91.2) (width 0.2) (layer "B.Cu") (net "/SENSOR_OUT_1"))
 (segment (start 119.365685 90.8) (end 87.12 90.8) (width 0.2) (layer "B.Cu") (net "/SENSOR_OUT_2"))
 (segment (start 87.12 90.8) (end 84.92 93) (width 0.2) (layer "B.Cu") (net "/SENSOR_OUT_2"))
 (segment (start 123.78 95.214315) (end 119.365685 90.8) (width 0.2) (layer "B.Cu") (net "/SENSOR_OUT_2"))
 (segment (start 123.78 97.32) (end 123.78 95.214315) (width 0.2) (layer "B.Cu") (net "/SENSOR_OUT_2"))
 (segment (start 126.32 97.32) (end 126.32 97.18863) (width 0.2) (layer "B.Cu") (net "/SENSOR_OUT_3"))
 (segment (start 84.98 90.4) (end 82.38 93) (width 0.2) (layer "B.Cu") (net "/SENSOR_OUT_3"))
 (segment (start 126.32 97.18863) (end 119.53137 90.4) (width 0.2) (layer "B.Cu") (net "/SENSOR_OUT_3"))
 (segment (start 119.53137 90.4) (end 84.98 90.4) (width 0.2) (layer "B.Cu") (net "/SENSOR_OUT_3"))
 (segment (start 121.54 90) (end 82.84 90) (width 0.2) (layer "B.Cu") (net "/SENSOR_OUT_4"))
 (segment (start 128.86 97.32) (end 121.54 90) (width 0.2) (layer "B.Cu") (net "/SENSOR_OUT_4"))
 (segment (start 82.84 90) (end 79.84 93) (width 0.2) (layer "B.Cu") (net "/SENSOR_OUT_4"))
 (segment (start 80.7 89.6) (end 77.3 93) (width 0.2) (layer "B.Cu") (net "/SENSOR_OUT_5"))
 (segment (start 123.68 89.6) (end 80.7 89.6) (width 0.2) (layer "B.Cu") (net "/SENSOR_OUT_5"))
 (segment (start 131.4 97.32) (end 123.68 89.6) (width 0.2) (layer "B.Cu") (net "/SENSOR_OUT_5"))
 (segment (start 125.82 89.2) (end 78.56 89.2) (width 0.2) (layer "B.Cu") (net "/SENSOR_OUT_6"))
 (segment (start 78.56 89.2) (end 74.76 93) (width 0.2) (layer "B.Cu") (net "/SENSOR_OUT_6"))
 (segment (start 133.94 97.32) (end 125.82 89.2) (width 0.2) (layer "B.Cu") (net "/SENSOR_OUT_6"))
 (segment (start 136.48 97.32) (end 127.96 88.8) (width 0.2) (layer "B.Cu") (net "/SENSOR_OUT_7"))
 (segment (start 76.42 88.8) (end 72.22 93) (width 0.2) (layer "B.Cu") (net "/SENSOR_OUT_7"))
 (segment (start 127.96 88.8) (end 76.42 88.8) (width 0.2) (layer "B.Cu") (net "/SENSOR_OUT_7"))
 (segment (start 130.1 88.4) (end 74.28 88.4) (width 0.2) (layer "B.Cu") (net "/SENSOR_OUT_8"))
 (segment (start 139.02 97.32) (end 130.1 88.4) (width 0.2) (layer "B.Cu") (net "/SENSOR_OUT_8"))
 (segment (start 74.28 88.4) (end 69.68 93) (width 0.2) (layer "B.Cu") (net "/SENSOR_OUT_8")))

